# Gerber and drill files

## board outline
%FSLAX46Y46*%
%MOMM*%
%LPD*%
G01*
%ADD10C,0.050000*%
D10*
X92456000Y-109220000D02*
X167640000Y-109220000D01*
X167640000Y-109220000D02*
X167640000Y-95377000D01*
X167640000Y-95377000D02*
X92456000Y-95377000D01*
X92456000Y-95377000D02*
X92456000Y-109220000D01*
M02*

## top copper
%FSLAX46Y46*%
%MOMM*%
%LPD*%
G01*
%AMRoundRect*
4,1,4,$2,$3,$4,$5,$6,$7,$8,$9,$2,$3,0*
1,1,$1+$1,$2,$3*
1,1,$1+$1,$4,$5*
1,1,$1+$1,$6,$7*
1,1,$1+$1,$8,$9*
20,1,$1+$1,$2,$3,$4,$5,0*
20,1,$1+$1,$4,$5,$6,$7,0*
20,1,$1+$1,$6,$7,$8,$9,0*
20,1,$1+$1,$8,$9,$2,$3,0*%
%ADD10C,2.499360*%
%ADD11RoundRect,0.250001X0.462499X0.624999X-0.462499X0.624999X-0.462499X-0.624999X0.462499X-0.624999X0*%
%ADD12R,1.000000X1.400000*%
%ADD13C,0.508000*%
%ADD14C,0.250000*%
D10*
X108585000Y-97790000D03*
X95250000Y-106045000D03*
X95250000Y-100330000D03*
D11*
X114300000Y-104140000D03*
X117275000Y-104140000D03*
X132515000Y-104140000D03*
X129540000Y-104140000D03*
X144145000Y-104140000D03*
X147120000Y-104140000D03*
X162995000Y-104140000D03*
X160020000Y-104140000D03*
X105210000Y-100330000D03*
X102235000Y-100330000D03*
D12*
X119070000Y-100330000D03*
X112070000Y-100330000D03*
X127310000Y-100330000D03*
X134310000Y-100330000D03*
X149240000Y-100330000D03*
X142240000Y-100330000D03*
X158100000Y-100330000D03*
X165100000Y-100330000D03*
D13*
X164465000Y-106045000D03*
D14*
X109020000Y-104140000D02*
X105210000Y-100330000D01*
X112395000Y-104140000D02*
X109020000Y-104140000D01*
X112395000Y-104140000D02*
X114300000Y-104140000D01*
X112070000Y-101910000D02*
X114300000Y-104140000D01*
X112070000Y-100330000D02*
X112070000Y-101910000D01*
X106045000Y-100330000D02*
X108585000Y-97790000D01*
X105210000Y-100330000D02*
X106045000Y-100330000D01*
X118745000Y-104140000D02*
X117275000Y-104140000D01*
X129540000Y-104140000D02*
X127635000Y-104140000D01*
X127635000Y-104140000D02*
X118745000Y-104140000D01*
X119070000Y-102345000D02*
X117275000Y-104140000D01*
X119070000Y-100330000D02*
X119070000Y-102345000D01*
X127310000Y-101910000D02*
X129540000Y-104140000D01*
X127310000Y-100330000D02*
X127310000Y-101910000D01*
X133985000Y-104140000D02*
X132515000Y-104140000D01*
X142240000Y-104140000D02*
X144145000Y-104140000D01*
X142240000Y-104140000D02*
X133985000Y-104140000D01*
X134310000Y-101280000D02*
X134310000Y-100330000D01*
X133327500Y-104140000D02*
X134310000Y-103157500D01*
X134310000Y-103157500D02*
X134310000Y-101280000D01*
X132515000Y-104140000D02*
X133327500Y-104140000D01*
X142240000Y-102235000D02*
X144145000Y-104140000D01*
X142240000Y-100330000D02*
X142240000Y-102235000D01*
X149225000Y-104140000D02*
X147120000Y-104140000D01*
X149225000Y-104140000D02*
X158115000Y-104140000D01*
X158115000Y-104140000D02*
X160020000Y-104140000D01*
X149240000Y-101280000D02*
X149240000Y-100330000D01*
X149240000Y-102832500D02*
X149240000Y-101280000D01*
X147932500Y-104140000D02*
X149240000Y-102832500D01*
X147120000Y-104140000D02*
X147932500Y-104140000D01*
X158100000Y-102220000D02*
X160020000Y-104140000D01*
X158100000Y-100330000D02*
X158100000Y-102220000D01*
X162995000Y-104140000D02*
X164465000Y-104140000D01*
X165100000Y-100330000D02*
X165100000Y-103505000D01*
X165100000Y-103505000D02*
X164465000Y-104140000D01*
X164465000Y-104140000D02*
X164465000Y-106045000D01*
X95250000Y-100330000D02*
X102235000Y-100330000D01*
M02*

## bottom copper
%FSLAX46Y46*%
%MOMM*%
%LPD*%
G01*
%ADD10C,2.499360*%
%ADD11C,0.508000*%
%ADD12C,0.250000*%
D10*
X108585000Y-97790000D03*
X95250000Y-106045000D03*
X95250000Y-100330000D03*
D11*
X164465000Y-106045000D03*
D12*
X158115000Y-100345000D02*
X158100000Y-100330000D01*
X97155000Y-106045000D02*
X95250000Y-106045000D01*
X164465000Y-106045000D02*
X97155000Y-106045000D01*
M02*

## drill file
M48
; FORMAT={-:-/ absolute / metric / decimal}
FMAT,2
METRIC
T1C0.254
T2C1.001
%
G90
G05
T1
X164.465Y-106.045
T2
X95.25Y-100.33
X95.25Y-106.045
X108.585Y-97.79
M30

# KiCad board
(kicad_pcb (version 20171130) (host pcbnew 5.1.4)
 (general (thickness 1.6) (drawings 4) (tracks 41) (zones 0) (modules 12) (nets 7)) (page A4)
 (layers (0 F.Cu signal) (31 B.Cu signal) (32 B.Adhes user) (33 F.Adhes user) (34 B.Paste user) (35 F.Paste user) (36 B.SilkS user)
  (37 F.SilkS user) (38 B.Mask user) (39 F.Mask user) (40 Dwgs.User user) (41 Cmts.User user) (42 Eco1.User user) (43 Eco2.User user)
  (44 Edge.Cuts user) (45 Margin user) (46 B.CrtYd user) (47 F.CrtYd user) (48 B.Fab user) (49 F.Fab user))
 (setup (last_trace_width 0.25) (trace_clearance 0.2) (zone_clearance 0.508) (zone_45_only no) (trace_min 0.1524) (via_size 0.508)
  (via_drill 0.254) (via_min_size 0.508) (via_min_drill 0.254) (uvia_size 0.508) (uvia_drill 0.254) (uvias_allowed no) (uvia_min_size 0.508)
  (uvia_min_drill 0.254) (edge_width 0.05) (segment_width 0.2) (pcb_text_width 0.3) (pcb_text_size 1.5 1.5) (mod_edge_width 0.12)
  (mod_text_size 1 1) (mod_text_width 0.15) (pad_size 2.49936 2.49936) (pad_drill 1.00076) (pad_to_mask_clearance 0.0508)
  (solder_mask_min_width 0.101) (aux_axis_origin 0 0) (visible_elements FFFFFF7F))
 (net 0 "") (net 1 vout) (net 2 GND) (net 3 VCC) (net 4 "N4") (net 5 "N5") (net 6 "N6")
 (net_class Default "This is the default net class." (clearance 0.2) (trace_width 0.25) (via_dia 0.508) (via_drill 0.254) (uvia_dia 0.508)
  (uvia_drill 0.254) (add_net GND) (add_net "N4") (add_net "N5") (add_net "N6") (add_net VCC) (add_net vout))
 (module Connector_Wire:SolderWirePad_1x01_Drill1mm (layer F.Cu) (at 108.585 97.79)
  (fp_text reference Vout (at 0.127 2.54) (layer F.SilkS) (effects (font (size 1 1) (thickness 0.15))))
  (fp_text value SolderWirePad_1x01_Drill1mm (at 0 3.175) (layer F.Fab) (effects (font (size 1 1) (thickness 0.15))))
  (pad 1 thru_hole circle (at 0 0) (size 2.49936 2.49936) (drill 1.00076) (layers *.Cu *.Mask) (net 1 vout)))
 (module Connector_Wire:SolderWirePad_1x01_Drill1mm (layer F.Cu) (at 95.25 106.045)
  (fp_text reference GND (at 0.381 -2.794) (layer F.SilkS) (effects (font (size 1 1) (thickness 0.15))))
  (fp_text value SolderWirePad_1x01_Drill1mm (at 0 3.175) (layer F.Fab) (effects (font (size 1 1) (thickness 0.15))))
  (pad 1 thru_hole circle (at 0 0) (size 2.49936 2.49936) (drill 1.00076) (layers *.Cu *.Mask) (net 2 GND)))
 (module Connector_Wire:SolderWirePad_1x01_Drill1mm (layer F.Cu) (at 95.25 100.33)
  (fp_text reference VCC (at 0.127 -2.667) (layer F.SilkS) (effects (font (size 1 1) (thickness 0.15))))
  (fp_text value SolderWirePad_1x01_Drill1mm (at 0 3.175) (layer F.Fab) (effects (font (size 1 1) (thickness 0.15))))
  (pad 1 thru_hole circle (at 0 0) (size 2.49936 2.49936) (drill 1.00076) (layers *.Cu *.Mask) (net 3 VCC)))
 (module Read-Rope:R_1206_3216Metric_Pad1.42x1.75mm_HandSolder (layer F.Cu) (at 115.7875 104.14 180)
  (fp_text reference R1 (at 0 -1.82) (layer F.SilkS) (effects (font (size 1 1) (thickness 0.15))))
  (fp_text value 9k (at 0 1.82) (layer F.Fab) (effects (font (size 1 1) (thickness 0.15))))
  (pad 2 smd roundrect (at 1.4875 0 180) (size 1.425 1.75) (layers F.Cu F.Paste F.Mask) (roundrect_rratio 0.175439) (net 1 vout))
  (pad 1 smd roundrect (at -1.4875 0 180) (size 1.425 1.75) (layers F.Cu F.Paste F.Mask) (roundrect_rratio 0.175439) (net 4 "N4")))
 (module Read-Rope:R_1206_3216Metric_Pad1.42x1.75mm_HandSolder (layer F.Cu) (at 131.0275 104.14 180)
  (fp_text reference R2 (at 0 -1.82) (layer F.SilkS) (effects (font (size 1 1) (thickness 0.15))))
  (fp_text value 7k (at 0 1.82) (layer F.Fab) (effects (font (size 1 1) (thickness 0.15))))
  (pad 1 smd roundrect (at -1.4875 0 180) (size 1.425 1.75) (layers F.Cu F.Paste F.Mask) (roundrect_rratio 0.175439) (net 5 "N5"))
  (pad 2 smd roundrect (at 1.4875 0 180) (size 1.425 1.75) (layers F.Cu F.Paste F.Mask) (roundrect_rratio 0.175439) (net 4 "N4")))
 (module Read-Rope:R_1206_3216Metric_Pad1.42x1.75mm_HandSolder (layer F.Cu) (at 145.6325 104.14 180)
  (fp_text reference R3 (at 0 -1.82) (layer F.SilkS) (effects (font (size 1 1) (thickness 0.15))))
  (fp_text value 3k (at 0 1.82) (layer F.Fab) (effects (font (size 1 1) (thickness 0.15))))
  (pad 2 smd roundrect (at 1.4875 0 180) (size 1.425 1.75) (layers F.Cu F.Paste F.Mask) (roundrect_rratio 0.175439) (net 5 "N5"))
  (pad 1 smd roundrect (at -1.4875 0 180) (size 1.425 1.75) (layers F.Cu F.Paste F.Mask) (roundrect_rratio 0.175439) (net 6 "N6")))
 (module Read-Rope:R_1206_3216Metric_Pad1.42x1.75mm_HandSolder (layer F.Cu) (at 161.5075 104.14 180)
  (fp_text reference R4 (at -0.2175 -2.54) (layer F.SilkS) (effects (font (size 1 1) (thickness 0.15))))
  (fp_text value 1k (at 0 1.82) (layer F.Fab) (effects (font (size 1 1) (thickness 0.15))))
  (pad 1 smd roundrect (at -1.4875 0 180) (size 1.425 1.75) (layers F.Cu F.Paste F.Mask) (roundrect_rratio 0.175439) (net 2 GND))
  (pad 2 smd roundrect (at 1.4875 0 180) (size 1.425 1.75) (layers F.Cu F.Paste F.Mask) (roundrect_rratio 0.175439) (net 6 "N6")))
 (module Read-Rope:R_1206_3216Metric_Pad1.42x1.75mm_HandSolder (layer F.Cu) (at 103.7225 100.33 180)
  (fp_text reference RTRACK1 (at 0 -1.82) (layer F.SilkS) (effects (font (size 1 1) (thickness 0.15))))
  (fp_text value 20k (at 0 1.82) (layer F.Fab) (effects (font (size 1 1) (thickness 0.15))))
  (pad 1 smd roundrect (at -1.4875 0 180) (size 1.425 1.75) (layers F.Cu F.Paste F.Mask) (roundrect_rratio 0.175439) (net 1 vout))
  (pad 2 smd roundrect (at 1.4875 0 180) (size 1.425 1.75) (layers F.Cu F.Paste F.Mask) (roundrect_rratio 0.175439) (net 3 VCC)))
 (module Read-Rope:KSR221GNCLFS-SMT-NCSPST (layer F.Cu) (at 115.57 100.33)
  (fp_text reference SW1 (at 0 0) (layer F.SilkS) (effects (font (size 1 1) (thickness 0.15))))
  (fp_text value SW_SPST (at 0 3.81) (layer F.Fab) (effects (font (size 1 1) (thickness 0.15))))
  (pad 2 smd rect (at 3.5 0) (size 1 1.4) (layers F.Cu F.Paste F.Mask) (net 4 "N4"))
  (pad 1 smd rect (at -3.5 0) (size 1 1.4) (layers F.Cu F.Paste F.Mask) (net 1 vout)))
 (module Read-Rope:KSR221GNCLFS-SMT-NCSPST (layer F.Cu) (at 130.81 100.33)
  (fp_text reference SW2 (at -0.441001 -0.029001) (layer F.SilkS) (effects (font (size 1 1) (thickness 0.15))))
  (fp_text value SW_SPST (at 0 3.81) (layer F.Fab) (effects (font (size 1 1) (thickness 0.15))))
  (pad 1 smd rect (at -3.5 0) (size 1 1.4) (layers F.Cu F.Paste F.Mask) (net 4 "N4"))
  (pad 2 smd rect (at 3.5 0) (size 1 1.4) (layers F.Cu F.Paste F.Mask) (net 5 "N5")))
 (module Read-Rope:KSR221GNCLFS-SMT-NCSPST (layer F.Cu) (at 145.74 100.33)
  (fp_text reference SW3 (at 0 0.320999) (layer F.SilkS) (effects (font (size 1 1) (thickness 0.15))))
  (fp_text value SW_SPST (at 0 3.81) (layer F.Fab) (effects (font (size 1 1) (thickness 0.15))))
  (pad 2 smd rect (at 3.5 0) (size 1 1.4) (layers F.Cu F.Paste F.Mask) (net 6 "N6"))
  (pad 1 smd rect (at -3.5 0) (size 1 1.4) (layers F.Cu F.Paste F.Mask) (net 5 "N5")))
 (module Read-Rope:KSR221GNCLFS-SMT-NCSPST (layer F.Cu) (at 161.6 100.33)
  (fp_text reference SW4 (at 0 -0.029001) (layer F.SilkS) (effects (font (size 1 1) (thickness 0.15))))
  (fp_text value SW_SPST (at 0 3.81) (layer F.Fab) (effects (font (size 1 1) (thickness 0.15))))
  (pad 1 smd rect (at -3.5 0) (size 1 1.4) (layers F.Cu F.Paste F.Mask) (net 6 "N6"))
  (pad 2 smd rect (at 3.5 0) (size 1 1.4) (layers F.Cu F.Paste F.Mask) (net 2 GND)))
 (gr_line (start 92.456 109.22) (end 167.64 109.22) (layer Edge.Cuts) (width 0.05))
 (gr_line (start 167.64 109.22) (end 167.64 95.377) (layer Edge.Cuts) (width 0.05))
 (gr_line (start 167.64 95.377) (end 92.456 95.377) (layer Edge.Cuts) (width 0.05))
 (gr_line (start 92.456 95.377) (end 92.456 109.22) (layer Edge.Cuts) (width 0.05))
 (segment (start 109.02 104.14) (end 105.21 100.33) (width 0.25) (layer F.Cu) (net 1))
 (segment (start 112.395 104.14) (end 109.02 104.14) (width 0.25) (layer F.Cu) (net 1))
 (segment (start 112.395 104.14) (end 114.3 104.14) (width 0.25) (layer F.Cu) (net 1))
 (segment (start 112.07 101.91) (end 114.3 104.14) (width 0.25) (layer F.Cu) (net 1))
 (segment (start 112.07 100.33) (end 112.07 101.91) (width 0.25) (layer F.Cu) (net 1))
 (segment (start 106.045 100.33) (end 108.585 97.79) (width 0.25) (layer F.Cu) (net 1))
 (segment (start 105.21 100.33) (end 106.045 100.33) (width 0.25) (layer F.Cu) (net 1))
 (segment (start 118.745 104.14) (end 117.275 104.14) (width 0.25) (layer F.Cu) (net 4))
 (segment (start 129.54 104.14) (end 127.635 104.14) (width 0.25) (layer F.Cu) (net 4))
 (segment (start 127.635 104.14) (end 118.745 104.14) (width 0.25) (layer F.Cu) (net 4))
 (segment (start 119.07 102.345) (end 117.275 104.14) (width 0.25) (layer F.Cu) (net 4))
 (segment (start 119.07 100.33) (end 119.07 102.345) (width 0.25) (layer F.Cu) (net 4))
 (segment (start 127.31 101.91) (end 129.54 104.14) (width 0.25) (layer F.Cu) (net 4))
 (segment (start 127.31 100.33) (end 127.31 101.91) (width 0.25) (layer F.Cu) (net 4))
 (segment (start 133.985 104.14) (end 132.515 104.14) (width 0.25) (layer F.Cu) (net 5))
 (segment (start 142.24 104.14) (end 144.145 104.14) (width 0.25) (layer F.Cu) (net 5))
 (segment (start 142.24 104.14) (end 133.985 104.14) (width 0.25) (layer F.Cu) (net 5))
 (segment (start 134.31 101.28) (end 134.31 100.33) (width 0.25) (layer F.Cu) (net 5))
 (segment (start 133.3275 104.14) (end 134.31 103.1575) (width 0.25) (layer F.Cu) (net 5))
 (segment (start 134.31 103.1575) (end 134.31 101.28) (width 0.25) (layer F.Cu) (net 5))
 (segment (start 132.515 104.14) (end 133.3275 104.14) (width 0.25) (layer F.Cu) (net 5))
 (segment (start 142.24 102.235) (end 144.145 104.14) (width 0.25) (layer F.Cu) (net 5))
 (segment (start 142.24 100.33) (end 142.24 102.235) (width 0.25) (layer F.Cu) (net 5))
 (segment (start 149.225 104.14) (end 147.12 104.14) (width 0.25) (layer F.Cu) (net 6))
 (segment (start 149.225 104.14) (end 158.115 104.14) (width 0.25) (layer F.Cu) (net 6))
 (segment (start 158.115 104.14) (end 160.02 104.14) (width 0.25) (layer F.Cu) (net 6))
 (segment (start 158.115 100.345) (end 158.1 100.33) (width 0.25) (layer B.Cu) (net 6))
 (segment (start 149.24 101.28) (end 149.24 100.33) (width 0.25) (layer F.Cu) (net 6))
 (segment (start 149.24 102.8325) (end 149.24 101.28) (width 0.25) (layer F.Cu) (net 6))
 (segment (start 147.9325 104.14) (end 149.24 102.8325) (width 0.25) (layer F.Cu) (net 6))
 (segment (start 147.12 104.14) (end 147.9325 104.14) (width 0.25) (layer F.Cu) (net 6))
 (segment (start 158.1 102.22) (end 160.02 104.14) (width 0.25) (layer F.Cu) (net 6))
 (segment (start 158.1 100.33) (end 158.1 102.22) (width 0.25) (layer F.Cu) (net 6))
 (segment (start 162.995 104.14) (end 164.465 104.14) (width 0.25) (layer F.Cu) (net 2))
 (segment (start 165.1 100.33) (end 165.1 103.505) (width 0.25) (layer F.Cu) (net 2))
 (segment (start 165.1 103.505) (end 164.465 104.14) (width 0.25) (layer F.Cu) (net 2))
 (via (at 164.465 106.045) (size 0.508) (drill 0.254) (layers F.Cu B.Cu) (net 2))
 (segment (start 164.465 104.14) (end 164.465 106.045) (width 0.25) (layer F.Cu) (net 2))
 (segment (start 97.155 106.045) (end 95.25 106.045) (width 0.25) (layer B.Cu) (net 2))
 (segment (start 164.465 106.045) (end 97.155 106.045) (width 0.25) (layer B.Cu) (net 2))
 (segment (start 95.25 100.33) (end 102.235 100.33) (width 0.25) (layer F.Cu) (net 3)))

